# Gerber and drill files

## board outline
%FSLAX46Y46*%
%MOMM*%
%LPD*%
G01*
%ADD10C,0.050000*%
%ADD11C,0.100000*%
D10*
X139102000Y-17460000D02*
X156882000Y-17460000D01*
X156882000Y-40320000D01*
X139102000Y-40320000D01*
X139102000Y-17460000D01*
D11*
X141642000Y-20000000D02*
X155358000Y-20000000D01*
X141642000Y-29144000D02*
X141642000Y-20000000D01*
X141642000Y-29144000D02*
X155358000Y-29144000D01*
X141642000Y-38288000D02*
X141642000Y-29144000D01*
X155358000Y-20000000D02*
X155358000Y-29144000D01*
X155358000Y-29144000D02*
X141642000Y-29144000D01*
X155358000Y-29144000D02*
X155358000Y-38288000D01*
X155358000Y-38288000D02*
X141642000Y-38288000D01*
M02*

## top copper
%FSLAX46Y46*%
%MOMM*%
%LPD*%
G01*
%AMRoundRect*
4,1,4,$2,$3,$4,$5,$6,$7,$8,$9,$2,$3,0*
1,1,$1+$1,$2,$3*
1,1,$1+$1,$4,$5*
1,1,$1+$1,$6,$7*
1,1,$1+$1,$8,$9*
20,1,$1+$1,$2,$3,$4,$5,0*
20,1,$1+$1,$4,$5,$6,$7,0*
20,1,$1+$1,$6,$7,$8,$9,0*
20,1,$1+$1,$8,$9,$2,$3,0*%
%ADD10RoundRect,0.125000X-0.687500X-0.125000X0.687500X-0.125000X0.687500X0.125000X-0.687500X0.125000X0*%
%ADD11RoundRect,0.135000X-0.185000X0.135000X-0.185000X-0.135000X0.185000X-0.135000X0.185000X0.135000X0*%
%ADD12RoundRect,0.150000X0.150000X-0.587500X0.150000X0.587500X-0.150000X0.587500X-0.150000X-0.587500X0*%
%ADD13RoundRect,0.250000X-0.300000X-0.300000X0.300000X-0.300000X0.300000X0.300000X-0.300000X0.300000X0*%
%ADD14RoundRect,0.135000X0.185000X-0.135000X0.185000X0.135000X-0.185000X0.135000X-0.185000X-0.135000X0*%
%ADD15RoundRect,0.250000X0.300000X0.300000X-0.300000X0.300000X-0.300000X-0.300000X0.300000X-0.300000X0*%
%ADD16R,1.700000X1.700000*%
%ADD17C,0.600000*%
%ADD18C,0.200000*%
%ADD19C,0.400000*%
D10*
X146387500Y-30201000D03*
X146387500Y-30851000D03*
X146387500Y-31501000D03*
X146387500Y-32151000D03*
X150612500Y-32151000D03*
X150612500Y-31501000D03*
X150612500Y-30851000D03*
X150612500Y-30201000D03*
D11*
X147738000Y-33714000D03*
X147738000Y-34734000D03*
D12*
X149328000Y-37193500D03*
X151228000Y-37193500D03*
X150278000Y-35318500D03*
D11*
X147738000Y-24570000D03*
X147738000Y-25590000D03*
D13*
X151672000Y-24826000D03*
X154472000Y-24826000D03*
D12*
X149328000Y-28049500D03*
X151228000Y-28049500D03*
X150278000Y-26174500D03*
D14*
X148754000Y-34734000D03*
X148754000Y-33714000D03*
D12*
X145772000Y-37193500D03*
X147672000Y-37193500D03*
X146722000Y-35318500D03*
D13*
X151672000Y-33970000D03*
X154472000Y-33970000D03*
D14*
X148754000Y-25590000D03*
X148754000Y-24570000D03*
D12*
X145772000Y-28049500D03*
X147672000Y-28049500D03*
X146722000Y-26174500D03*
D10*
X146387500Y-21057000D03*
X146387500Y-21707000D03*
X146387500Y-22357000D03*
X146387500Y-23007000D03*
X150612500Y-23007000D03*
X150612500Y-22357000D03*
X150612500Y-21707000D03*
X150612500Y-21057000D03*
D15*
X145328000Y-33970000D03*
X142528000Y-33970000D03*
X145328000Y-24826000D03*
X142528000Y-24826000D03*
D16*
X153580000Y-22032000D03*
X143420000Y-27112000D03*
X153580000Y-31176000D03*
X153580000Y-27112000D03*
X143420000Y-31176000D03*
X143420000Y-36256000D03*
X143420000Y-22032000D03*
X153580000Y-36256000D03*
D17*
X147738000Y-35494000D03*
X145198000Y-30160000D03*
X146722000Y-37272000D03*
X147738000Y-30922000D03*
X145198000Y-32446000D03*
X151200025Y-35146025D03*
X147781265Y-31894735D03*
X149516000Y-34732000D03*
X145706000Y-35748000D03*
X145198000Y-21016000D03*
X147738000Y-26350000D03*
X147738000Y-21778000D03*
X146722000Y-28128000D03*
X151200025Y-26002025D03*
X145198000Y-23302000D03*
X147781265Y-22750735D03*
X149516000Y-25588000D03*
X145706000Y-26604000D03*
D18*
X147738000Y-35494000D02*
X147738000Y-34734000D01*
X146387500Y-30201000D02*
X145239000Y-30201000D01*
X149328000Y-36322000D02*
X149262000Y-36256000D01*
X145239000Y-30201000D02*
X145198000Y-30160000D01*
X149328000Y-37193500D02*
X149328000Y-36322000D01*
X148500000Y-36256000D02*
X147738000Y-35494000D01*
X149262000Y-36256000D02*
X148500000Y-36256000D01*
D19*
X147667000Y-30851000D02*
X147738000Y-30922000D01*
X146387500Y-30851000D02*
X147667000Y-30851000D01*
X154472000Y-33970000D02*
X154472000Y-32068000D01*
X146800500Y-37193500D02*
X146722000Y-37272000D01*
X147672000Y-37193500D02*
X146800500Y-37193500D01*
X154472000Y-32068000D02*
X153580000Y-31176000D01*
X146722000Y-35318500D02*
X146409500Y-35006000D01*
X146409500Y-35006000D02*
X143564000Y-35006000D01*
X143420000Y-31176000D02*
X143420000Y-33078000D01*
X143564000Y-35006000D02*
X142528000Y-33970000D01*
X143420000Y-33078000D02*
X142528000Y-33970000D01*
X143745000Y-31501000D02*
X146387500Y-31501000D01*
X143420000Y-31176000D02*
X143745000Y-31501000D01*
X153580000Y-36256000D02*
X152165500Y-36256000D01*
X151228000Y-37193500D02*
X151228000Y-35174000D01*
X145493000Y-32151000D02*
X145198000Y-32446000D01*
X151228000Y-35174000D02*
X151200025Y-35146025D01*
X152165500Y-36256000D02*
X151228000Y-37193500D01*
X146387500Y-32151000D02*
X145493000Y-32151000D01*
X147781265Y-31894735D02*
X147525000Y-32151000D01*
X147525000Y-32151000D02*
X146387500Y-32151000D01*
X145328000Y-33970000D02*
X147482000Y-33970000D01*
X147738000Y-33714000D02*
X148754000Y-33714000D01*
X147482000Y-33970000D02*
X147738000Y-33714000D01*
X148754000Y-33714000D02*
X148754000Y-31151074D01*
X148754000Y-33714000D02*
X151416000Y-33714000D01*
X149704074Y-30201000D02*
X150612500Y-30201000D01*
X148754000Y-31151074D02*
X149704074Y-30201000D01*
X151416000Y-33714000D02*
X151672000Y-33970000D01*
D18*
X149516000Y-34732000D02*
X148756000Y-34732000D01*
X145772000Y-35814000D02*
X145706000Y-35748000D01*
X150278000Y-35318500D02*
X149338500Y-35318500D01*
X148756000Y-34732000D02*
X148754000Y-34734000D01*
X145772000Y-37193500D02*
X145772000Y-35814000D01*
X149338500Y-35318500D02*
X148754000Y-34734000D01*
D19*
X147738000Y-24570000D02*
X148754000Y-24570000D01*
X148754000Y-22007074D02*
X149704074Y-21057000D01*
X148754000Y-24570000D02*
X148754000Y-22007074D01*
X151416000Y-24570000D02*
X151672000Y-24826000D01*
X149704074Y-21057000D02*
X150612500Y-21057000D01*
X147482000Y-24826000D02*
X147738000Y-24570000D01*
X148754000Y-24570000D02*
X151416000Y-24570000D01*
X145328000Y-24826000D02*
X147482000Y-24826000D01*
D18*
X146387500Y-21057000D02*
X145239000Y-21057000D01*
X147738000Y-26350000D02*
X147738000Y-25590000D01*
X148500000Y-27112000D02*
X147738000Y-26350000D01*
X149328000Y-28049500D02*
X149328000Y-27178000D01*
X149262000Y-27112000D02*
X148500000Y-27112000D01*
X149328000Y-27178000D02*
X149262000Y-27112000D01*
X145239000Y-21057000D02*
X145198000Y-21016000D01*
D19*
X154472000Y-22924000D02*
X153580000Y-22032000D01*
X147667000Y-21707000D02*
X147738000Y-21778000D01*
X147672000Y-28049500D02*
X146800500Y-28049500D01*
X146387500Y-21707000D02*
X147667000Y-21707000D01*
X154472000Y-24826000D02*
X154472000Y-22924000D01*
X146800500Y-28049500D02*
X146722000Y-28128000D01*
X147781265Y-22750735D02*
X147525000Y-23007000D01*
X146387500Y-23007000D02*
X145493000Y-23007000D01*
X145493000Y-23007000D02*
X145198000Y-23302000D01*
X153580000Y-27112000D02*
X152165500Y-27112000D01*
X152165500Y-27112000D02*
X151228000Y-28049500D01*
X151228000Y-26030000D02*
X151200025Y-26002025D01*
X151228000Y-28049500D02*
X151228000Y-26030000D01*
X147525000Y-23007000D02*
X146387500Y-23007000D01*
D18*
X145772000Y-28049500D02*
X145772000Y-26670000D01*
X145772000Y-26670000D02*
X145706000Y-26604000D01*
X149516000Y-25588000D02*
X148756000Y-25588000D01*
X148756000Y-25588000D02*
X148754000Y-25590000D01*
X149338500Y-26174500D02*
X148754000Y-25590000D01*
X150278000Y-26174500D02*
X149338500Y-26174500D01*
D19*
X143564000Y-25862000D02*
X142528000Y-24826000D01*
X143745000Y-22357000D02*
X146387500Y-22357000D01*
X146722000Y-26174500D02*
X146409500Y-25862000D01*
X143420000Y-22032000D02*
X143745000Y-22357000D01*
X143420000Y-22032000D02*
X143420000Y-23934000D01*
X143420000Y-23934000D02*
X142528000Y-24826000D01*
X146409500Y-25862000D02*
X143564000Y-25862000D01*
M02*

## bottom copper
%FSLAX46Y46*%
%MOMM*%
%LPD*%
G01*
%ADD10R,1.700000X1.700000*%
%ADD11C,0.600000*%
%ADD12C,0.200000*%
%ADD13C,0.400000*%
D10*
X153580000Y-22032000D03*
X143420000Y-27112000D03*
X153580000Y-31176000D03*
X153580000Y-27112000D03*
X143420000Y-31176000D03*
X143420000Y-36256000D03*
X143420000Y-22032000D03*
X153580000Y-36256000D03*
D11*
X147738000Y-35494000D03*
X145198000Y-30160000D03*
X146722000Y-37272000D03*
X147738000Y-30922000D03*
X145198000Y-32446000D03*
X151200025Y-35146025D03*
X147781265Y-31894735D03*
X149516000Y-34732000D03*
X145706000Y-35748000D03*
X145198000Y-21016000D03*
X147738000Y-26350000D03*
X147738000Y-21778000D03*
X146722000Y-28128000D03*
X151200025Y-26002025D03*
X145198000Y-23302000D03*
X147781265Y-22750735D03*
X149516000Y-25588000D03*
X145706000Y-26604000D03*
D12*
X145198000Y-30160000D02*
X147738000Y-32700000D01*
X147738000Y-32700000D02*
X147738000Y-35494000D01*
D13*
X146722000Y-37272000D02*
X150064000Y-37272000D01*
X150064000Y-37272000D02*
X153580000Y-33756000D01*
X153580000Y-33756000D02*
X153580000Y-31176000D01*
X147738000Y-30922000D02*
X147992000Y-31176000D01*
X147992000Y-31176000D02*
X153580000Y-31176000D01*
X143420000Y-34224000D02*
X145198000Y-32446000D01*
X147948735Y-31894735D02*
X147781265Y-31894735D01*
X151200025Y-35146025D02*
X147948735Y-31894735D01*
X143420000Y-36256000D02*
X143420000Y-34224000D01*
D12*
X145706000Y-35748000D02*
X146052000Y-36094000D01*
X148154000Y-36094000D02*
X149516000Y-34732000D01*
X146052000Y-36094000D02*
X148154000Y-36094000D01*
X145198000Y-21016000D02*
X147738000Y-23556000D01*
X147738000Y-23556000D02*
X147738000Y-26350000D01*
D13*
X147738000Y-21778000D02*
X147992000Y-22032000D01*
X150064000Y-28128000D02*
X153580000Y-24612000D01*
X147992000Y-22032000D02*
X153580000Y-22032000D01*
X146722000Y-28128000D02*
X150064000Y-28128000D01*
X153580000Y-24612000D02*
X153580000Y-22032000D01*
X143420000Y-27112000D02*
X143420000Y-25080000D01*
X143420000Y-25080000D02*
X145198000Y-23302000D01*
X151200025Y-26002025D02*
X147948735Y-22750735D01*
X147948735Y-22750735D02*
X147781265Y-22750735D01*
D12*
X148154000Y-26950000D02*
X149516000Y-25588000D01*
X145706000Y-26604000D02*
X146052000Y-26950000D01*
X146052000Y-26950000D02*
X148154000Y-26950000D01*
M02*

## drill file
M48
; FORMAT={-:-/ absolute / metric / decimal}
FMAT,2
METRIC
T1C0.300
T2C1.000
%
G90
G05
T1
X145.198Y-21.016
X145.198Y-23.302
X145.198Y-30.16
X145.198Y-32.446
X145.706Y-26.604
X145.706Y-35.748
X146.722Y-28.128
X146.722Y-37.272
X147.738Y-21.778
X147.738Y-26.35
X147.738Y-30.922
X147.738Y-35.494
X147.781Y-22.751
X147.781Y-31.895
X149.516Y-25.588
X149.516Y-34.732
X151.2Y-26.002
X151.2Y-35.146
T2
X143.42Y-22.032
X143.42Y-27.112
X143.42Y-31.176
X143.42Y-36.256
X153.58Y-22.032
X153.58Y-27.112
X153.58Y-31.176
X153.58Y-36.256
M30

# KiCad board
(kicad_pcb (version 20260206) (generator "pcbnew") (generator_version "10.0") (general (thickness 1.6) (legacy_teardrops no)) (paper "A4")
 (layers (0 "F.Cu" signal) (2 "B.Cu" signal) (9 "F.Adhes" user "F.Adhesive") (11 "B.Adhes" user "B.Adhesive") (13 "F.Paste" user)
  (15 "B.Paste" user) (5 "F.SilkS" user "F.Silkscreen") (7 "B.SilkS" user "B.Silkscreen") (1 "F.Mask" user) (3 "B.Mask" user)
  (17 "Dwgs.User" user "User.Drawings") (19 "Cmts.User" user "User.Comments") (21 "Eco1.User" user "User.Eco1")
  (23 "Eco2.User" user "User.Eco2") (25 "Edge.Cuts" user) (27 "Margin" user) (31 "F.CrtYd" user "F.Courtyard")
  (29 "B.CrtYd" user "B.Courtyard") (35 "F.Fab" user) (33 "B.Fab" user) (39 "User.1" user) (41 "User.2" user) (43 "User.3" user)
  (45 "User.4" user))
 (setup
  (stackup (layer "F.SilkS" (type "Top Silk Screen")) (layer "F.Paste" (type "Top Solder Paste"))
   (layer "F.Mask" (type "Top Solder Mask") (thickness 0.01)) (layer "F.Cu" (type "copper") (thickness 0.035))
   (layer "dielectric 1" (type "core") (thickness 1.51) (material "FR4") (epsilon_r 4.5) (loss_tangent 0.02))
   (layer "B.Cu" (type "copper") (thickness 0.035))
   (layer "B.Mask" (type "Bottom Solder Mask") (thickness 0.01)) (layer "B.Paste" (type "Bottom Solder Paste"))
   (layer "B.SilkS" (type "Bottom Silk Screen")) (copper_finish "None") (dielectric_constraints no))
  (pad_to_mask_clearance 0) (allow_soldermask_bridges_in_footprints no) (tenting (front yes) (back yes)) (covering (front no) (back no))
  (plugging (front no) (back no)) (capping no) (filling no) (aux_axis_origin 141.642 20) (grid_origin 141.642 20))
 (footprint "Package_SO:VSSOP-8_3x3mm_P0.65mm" (layer "F.Cu") (at 148.5 31.176)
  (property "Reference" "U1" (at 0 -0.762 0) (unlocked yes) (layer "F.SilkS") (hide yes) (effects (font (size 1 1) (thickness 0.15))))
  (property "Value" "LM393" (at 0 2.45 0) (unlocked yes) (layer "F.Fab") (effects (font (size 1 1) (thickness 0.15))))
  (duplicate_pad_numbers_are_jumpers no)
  (pad "1" smd roundrect (at -2.1125 -0.975) (size 1.625 0.5) (layers "F.Cu" "F.Mask" "F.Paste") (roundrect_rratio 0.25)
   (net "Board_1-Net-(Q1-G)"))
  (pad "2" smd roundrect (at -2.1125 -0.325) (size 1.625 0.5) (layers "F.Cu" "F.Mask" "F.Paste") (roundrect_rratio 0.25) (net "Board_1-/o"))
  (pad "3" smd roundrect (at -2.1125 0.325) (size 1.625 0.5) (layers "F.Cu" "F.Mask" "F.Paste") (roundrect_rratio 0.25) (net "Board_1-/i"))
  (pad "4" smd roundrect (at -2.1125 0.975) (size 1.625 0.5) (layers "F.Cu" "F.Mask" "F.Paste") (roundrect_rratio 0.25) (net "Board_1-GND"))
  (pad "5" smd roundrect (at 2.1125 0.975) (size 1.625 0.5) (layers "F.Cu" "F.Mask" "F.Paste") (roundrect_rratio 0.25)
   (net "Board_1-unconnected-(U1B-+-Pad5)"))
  (pad "6" smd roundrect (at 2.1125 0.325) (size 1.625 0.5) (layers "F.Cu" "F.Mask" "F.Paste") (roundrect_rratio 0.25)
   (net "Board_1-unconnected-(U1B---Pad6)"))
  (pad "7" smd roundrect (at 2.1125 -0.325) (size 1.625 0.5) (layers "F.Cu" "F.Mask" "F.Paste") (roundrect_rratio 0.25)
   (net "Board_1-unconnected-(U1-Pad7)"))
  (pad "8" smd roundrect (at 2.1125 -0.975) (size 1.625 0.5) (layers "F.Cu" "F.Mask" "F.Paste") (roundrect_rratio 0.25) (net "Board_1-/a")))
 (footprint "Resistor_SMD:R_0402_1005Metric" (layer "F.Cu") (at 147.738 34.224 -90)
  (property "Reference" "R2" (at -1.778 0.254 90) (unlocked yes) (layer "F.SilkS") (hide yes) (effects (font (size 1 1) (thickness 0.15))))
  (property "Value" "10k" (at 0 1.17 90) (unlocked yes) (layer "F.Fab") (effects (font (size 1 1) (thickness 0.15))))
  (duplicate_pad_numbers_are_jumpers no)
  (pad "1" smd roundrect (at -0.51 0 270) (size 0.54 0.64) (layers "F.Cu" "F.Mask" "F.Paste") (roundrect_rratio 0.25) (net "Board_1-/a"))
  (pad "2" smd roundrect (at 0.51 0 270) (size 0.54 0.64) (layers "F.Cu" "F.Mask" "F.Paste") (roundrect_rratio 0.25)
   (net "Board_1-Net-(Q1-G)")))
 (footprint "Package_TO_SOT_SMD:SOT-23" (layer "F.Cu") (at 150.278 36.256 90)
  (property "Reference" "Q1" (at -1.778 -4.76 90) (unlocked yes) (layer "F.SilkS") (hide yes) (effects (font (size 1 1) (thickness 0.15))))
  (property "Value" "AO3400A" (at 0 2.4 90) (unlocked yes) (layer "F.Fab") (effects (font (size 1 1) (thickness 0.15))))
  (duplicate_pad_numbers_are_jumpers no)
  (pad "1" smd roundrect (at -0.9375 -0.95 90) (size 1.475 0.6) (layers "F.Cu" "F.Mask" "F.Paste") (roundrect_rratio 0.25)
   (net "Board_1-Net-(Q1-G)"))
  (pad "2" smd roundrect (at -0.9375 0.95 90) (size 1.475 0.6) (layers "F.Cu" "F.Mask" "F.Paste") (roundrect_rratio 0.25)
   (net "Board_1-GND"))
  (pad "3" smd roundrect (at 0.9375 0 90) (size 1.475 0.6) (layers "F.Cu" "F.Mask" "F.Paste") (roundrect_rratio 0.25)
   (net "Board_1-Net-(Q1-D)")))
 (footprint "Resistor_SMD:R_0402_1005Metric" (layer "F.Cu") (at 147.738 25.08 -90)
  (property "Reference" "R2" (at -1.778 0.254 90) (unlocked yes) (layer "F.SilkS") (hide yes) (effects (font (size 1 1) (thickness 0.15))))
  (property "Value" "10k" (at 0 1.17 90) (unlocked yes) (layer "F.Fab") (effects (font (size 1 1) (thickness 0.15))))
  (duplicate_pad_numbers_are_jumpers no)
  (pad "1" smd roundrect (at -0.51 0 270) (size 0.54 0.64) (layers "F.Cu" "F.Mask" "F.Paste") (roundrect_rratio 0.25) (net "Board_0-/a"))
  (pad "2" smd roundrect (at 0.51 0 270) (size 0.54 0.64) (layers "F.Cu" "F.Mask" "F.Paste") (roundrect_rratio 0.25)
   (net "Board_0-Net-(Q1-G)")))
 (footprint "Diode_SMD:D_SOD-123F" (layer "F.Cu") (at 153.072 24.826)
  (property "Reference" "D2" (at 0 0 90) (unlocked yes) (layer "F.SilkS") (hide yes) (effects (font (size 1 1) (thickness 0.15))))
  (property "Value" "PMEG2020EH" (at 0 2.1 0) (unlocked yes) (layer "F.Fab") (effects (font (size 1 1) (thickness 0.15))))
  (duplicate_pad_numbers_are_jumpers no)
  (pad "1" smd roundrect (at -1.4 0) (size 1.1 1.1) (layers "F.Cu" "F.Mask" "F.Paste") (roundrect_rratio 0.2272727273) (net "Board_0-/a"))
  (pad "2" smd roundrect (at 1.4 0) (size 1.1 1.1) (layers "F.Cu" "F.Mask" "F.Paste") (roundrect_rratio 0.2272727273) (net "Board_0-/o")))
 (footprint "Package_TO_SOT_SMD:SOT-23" (layer "F.Cu") (at 150.278 27.112 90)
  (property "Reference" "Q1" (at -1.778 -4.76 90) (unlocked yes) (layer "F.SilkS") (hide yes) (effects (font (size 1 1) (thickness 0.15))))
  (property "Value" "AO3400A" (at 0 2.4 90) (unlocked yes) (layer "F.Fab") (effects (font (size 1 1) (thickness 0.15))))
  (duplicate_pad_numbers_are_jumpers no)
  (pad "1" smd roundrect (at -0.9375 -0.95 90) (size 1.475 0.6) (layers "F.Cu" "F.Mask" "F.Paste") (roundrect_rratio 0.25)
   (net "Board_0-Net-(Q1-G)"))
  (pad "2" smd roundrect (at -0.9375 0.95 90) (size 1.475 0.6) (layers "F.Cu" "F.Mask" "F.Paste") (roundrect_rratio 0.25)
   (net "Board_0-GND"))
  (pad "3" smd roundrect (at 0.9375 0 90) (size 1.475 0.6) (layers "F.Cu" "F.Mask" "F.Paste") (roundrect_rratio 0.25)
   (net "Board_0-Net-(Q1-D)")))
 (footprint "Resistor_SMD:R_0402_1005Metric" (layer "F.Cu") (at 148.754 34.224 90)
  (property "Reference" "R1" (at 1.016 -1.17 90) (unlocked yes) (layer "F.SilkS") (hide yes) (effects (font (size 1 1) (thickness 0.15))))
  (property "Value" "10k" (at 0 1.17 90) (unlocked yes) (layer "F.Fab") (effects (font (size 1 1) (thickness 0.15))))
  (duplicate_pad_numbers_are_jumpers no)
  (pad "1" smd roundrect (at -0.51 0 90) (size 0.54 0.64) (layers "F.Cu" "F.Mask" "F.Paste") (roundrect_rratio 0.25)
   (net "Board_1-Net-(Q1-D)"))
  (pad "2" smd roundrect (at 0.51 0 90) (size 0.54 0.64) (layers "F.Cu" "F.Mask" "F.Paste") (roundrect_rratio 0.25) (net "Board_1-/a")))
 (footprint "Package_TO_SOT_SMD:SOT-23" (layer "F.Cu") (at 146.722 36.256 90)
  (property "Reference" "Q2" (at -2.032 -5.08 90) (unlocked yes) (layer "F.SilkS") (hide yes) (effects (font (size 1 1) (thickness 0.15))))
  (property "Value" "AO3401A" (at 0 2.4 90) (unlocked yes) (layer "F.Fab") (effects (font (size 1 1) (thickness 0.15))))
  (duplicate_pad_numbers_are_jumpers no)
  (pad "1" smd roundrect (at -0.9375 -0.95 90) (size 1.475 0.6) (layers "F.Cu" "F.Mask" "F.Paste") (roundrect_rratio 0.25)
   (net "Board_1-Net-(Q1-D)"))
  (pad "2" smd roundrect (at -0.9375 0.95 90) (size 1.475 0.6) (layers "F.Cu" "F.Mask" "F.Paste") (roundrect_rratio 0.25) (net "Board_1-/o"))
  (pad "3" smd roundrect (at 0.9375 0 90) (size 1.475 0.6) (layers "F.Cu" "F.Mask" "F.Paste") (roundrect_rratio 0.25) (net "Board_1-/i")))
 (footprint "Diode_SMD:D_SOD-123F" (layer "F.Cu") (at 153.072 33.97)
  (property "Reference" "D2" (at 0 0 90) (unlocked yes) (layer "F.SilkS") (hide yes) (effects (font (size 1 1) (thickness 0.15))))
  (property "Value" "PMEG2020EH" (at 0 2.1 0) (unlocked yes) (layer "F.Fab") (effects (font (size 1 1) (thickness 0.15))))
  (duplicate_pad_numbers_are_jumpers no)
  (pad "1" smd roundrect (at -1.4 0) (size 1.1 1.1) (layers "F.Cu" "F.Mask" "F.Paste") (roundrect_rratio 0.2272727273) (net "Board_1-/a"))
  (pad "2" smd roundrect (at 1.4 0) (size 1.1 1.1) (layers "F.Cu" "F.Mask" "F.Paste") (roundrect_rratio 0.2272727273) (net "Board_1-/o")))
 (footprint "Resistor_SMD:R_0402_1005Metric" (layer "F.Cu") (at 148.754 25.08 90)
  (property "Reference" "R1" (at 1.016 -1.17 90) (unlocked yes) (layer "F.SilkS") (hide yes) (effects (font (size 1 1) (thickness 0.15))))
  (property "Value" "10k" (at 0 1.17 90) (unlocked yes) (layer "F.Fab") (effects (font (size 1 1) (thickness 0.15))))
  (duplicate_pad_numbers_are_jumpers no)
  (pad "1" smd roundrect (at -0.51 0 90) (size 0.54 0.64) (layers "F.Cu" "F.Mask" "F.Paste") (roundrect_rratio 0.25)
   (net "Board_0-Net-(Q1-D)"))
  (pad "2" smd roundrect (at 0.51 0 90) (size 0.54 0.64) (layers "F.Cu" "F.Mask" "F.Paste") (roundrect_rratio 0.25) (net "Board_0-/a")))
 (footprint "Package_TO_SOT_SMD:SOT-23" (layer "F.Cu") (at 146.722 27.112 90)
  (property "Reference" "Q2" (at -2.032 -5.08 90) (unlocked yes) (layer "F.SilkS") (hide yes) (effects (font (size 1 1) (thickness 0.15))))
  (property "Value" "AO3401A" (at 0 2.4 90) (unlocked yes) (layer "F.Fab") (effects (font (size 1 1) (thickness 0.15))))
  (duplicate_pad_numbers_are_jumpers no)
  (pad "1" smd roundrect (at -0.9375 -0.95 90) (size 1.475 0.6) (layers "F.Cu" "F.Mask" "F.Paste") (roundrect_rratio 0.25)
   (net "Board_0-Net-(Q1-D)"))
  (pad "2" smd roundrect (at -0.9375 0.95 90) (size 1.475 0.6) (layers "F.Cu" "F.Mask" "F.Paste") (roundrect_rratio 0.25) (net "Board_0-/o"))
  (pad "3" smd roundrect (at 0.9375 0 90) (size 1.475 0.6) (layers "F.Cu" "F.Mask" "F.Paste") (roundrect_rratio 0.25) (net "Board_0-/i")))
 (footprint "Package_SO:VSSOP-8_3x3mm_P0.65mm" (layer "F.Cu") (at 148.5 22.032)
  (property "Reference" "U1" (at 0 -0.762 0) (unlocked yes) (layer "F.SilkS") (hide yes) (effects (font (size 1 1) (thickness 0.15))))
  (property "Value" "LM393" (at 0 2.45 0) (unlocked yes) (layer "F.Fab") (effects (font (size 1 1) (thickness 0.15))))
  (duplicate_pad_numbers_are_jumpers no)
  (pad "1" smd roundrect (at -2.1125 -0.975) (size 1.625 0.5) (layers "F.Cu" "F.Mask" "F.Paste") (roundrect_rratio 0.25)
   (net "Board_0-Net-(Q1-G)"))
  (pad "2" smd roundrect (at -2.1125 -0.325) (size 1.625 0.5) (layers "F.Cu" "F.Mask" "F.Paste") (roundrect_rratio 0.25) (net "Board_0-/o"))
  (pad "3" smd roundrect (at -2.1125 0.325) (size 1.625 0.5) (layers "F.Cu" "F.Mask" "F.Paste") (roundrect_rratio 0.25) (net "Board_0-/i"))
  (pad "4" smd roundrect (at -2.1125 0.975) (size 1.625 0.5) (layers "F.Cu" "F.Mask" "F.Paste") (roundrect_rratio 0.25) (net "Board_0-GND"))
  (pad "5" smd roundrect (at 2.1125 0.975) (size 1.625 0.5) (layers "F.Cu" "F.Mask" "F.Paste") (roundrect_rratio 0.25)
   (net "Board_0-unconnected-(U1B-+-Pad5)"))
  (pad "6" smd roundrect (at 2.1125 0.325) (size 1.625 0.5) (layers "F.Cu" "F.Mask" "F.Paste") (roundrect_rratio 0.25)
   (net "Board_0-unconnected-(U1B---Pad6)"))
  (pad "7" smd roundrect (at 2.1125 -0.325) (size 1.625 0.5) (layers "F.Cu" "F.Mask" "F.Paste") (roundrect_rratio 0.25)
   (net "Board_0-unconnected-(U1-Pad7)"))
  (pad "8" smd roundrect (at 2.1125 -0.975) (size 1.625 0.5) (layers "F.Cu" "F.Mask" "F.Paste") (roundrect_rratio 0.25) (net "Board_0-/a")))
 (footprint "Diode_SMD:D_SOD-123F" (layer "F.Cu") (at 143.928 33.97 180)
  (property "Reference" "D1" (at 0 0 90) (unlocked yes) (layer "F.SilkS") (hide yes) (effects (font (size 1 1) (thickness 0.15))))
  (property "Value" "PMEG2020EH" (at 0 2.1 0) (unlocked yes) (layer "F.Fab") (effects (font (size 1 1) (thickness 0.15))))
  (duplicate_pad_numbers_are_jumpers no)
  (pad "1" smd roundrect (at -1.4 0 180) (size 1.1 1.1) (layers "F.Cu" "F.Mask" "F.Paste") (roundrect_rratio 0.2272727273)
   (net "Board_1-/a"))
  (pad "2" smd roundrect (at 1.4 0 180) (size 1.1 1.1) (layers "F.Cu" "F.Mask" "F.Paste") (roundrect_rratio 0.2272727273) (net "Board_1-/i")))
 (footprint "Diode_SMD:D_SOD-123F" (layer "F.Cu") (at 143.928 24.826 180)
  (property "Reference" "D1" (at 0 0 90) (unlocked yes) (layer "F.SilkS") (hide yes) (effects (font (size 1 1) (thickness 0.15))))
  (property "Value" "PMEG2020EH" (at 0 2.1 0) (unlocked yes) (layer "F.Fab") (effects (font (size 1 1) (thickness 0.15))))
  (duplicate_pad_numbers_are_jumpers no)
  (pad "1" smd roundrect (at -1.4 0 180) (size 1.1 1.1) (layers "F.Cu" "F.Mask" "F.Paste") (roundrect_rratio 0.2272727273)
   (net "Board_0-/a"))
  (pad "2" smd roundrect (at 1.4 0 180) (size 1.1 1.1) (layers "F.Cu" "F.Mask" "F.Paste") (roundrect_rratio 0.2272727273) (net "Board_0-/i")))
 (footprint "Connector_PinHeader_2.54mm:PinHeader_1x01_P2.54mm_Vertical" (layer "B.Cu") (at 153.58 22.032 180)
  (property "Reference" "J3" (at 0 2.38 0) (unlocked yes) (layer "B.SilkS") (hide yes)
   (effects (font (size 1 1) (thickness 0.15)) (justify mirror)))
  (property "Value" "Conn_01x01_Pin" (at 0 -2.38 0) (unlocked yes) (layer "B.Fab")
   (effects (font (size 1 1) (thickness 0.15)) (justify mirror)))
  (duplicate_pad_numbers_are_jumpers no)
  (pad "1" thru_hole rect (at 0 0 180) (size 1.7 1.7) (drill 1) (layers "*.Cu" "*.Mask") (remove_unused_layers no) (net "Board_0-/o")))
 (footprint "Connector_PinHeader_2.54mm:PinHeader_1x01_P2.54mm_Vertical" (layer "B.Cu") (at 143.42 27.112 180)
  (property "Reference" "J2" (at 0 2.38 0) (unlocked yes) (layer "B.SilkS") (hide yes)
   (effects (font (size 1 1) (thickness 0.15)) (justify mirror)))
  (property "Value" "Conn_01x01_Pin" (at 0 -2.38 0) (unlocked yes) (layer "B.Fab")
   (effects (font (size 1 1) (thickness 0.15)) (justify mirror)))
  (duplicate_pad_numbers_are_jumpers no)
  (pad "1" thru_hole rect (at 0 0 180) (size 1.7 1.7) (drill 1) (layers "*.Cu" "*.Mask") (remove_unused_layers no) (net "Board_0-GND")))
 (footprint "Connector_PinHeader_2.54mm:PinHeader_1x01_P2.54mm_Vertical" (layer "B.Cu") (at 153.58 31.176 180)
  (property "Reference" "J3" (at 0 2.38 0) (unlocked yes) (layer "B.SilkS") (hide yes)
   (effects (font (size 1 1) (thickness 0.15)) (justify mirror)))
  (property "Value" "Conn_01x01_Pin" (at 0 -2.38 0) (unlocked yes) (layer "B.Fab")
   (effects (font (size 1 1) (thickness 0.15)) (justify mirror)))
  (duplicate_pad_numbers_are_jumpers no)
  (pad "1" thru_hole rect (at 0 0 180) (size 1.7 1.7) (drill 1) (layers "*.Cu" "*.Mask") (remove_unused_layers no) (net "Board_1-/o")))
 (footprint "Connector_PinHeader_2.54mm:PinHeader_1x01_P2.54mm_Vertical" (layer "B.Cu") (at 153.58 27.112 180)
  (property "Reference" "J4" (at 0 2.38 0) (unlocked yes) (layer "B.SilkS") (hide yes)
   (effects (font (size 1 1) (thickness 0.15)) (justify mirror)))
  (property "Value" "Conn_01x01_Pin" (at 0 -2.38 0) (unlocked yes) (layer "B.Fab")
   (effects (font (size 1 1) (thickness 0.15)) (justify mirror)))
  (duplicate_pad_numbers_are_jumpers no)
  (pad "1" thru_hole rect (at 0 0 180) (size 1.7 1.7) (drill 1) (layers "*.Cu" "*.Mask") (remove_unused_layers no) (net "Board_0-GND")))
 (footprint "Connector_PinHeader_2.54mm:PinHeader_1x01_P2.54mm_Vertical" (layer "B.Cu") (at 143.42 31.176 180)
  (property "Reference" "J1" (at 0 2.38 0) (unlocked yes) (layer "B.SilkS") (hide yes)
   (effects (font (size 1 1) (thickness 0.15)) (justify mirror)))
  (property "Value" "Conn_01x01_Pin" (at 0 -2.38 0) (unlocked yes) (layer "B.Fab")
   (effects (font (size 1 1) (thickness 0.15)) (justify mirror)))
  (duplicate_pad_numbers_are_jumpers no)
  (pad "1" thru_hole rect (at 0 0 180) (size 1.7 1.7) (drill 1) (layers "*.Cu" "*.Mask") (remove_unused_layers no) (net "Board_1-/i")))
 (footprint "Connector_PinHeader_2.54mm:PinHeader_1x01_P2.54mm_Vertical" (layer "B.Cu") (at 143.42 36.256 180)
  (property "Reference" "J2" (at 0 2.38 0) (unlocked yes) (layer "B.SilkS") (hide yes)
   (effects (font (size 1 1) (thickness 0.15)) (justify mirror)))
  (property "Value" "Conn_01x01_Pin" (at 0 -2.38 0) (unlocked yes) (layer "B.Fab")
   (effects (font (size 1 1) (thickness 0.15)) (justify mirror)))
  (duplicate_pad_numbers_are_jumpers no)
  (pad "1" thru_hole rect (at 0 0 180) (size 1.7 1.7) (drill 1) (layers "*.Cu" "*.Mask") (remove_unused_layers no) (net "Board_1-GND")))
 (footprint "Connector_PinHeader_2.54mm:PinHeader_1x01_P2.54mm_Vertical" (layer "B.Cu") (at 143.42 22.032 180)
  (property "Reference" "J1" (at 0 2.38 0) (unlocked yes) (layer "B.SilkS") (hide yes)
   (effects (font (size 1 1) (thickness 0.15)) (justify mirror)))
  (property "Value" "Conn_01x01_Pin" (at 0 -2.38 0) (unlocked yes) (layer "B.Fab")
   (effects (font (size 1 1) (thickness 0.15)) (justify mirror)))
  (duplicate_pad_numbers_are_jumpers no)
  (pad "1" thru_hole rect (at 0 0 180) (size 1.7 1.7) (drill 1) (layers "*.Cu" "*.Mask") (remove_unused_layers no) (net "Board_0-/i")))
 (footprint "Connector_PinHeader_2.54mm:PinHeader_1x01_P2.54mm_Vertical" (layer "B.Cu") (at 153.58 36.256 180)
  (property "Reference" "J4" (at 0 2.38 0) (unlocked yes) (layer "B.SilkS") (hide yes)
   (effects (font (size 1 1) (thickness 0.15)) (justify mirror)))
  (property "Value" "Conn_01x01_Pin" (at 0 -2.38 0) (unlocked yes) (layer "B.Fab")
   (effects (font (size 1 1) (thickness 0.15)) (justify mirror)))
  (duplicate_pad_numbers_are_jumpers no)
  (pad "1" thru_hole rect (at 0 0 180) (size 1.7 1.7) (drill 1) (layers "*.Cu" "*.Mask") (remove_unused_layers no) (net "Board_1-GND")))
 (gr_rect (start 139.102 17.46) (end 156.882 40.32) (stroke (width 0.05) (type default)) (fill no) (layer "Edge.Cuts"))
 (gr_line (start 141.642 20) (end 155.358 20) (stroke (width 0.1) (type default)) (layer "Edge.Cuts"))
 (gr_line (start 141.642 29.144) (end 141.642 20) (stroke (width 0.1) (type default)) (layer "Edge.Cuts"))
 (gr_line (start 141.642 29.144) (end 155.358 29.144) (stroke (width 0.1) (type default)) (layer "Edge.Cuts"))
 (gr_line (start 141.642 38.288) (end 141.642 29.144) (stroke (width 0.1) (type default)) (layer "Edge.Cuts"))
 (gr_line (start 155.358 20) (end 155.358 29.144) (stroke (width 0.1) (type default)) (layer "Edge.Cuts"))
 (gr_line (start 155.358 29.144) (end 141.642 29.144) (stroke (width 0.1) (type default)) (layer "Edge.Cuts"))
 (gr_line (start 155.358 29.144) (end 155.358 38.288) (stroke (width 0.1) (type default)) (layer "Edge.Cuts"))
 (gr_line (start 155.358 38.288) (end 141.642 38.288) (stroke (width 0.1) (type default)) (layer "Edge.Cuts"))
 (segment (start 147.738 35.494) (end 147.738 34.734) (width 0.2) (layer "F.Cu") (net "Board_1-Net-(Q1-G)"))
 (segment (start 146.3875 30.201) (end 145.239 30.201) (width 0.2) (layer "F.Cu") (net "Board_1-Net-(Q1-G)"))
 (segment (start 149.328 36.322) (end 149.262 36.256) (width 0.2) (layer "F.Cu") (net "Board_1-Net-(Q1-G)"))
 (segment (start 145.239 30.201) (end 145.198 30.16) (width 0.2) (layer "F.Cu") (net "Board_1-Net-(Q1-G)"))
 (segment (start 149.328 37.1935) (end 149.328 36.322) (width 0.2) (layer "F.Cu") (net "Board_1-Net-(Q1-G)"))
 (segment (start 148.5 36.256) (end 147.738 35.494) (width 0.2) (layer "F.Cu") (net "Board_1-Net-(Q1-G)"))
 (segment (start 149.262 36.256) (end 148.5 36.256) (width 0.2) (layer "F.Cu") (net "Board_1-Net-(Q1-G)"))
 (via (at 147.738 35.494) (size 0.6) (drill 0.3) (layers "F.Cu" "B.Cu") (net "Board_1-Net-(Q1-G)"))
 (via (at 145.198 30.16) (size 0.6) (drill 0.3) (layers "F.Cu" "B.Cu") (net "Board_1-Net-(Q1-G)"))
 (segment (start 145.198 30.16) (end 147.738 32.7) (width 0.2) (layer "B.Cu") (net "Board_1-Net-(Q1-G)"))
 (segment (start 147.738 32.7) (end 147.738 35.494) (width 0.2) (layer "B.Cu") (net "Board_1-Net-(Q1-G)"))
 (segment (start 147.667 30.851) (end 147.738 30.922) (width 0.4) (layer "F.Cu") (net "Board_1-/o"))
 (segment (start 146.3875 30.851) (end 147.667 30.851) (width 0.4) (layer "F.Cu") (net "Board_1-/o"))
 (segment (start 154.472 33.97) (end 154.472 32.068) (width 0.4) (layer "F.Cu") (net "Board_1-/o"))
 (segment (start 146.8005 37.1935) (end 146.722 37.272) (width 0.4) (layer "F.Cu") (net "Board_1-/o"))
 (segment (start 147.672 37.1935) (end 146.8005 37.1935) (width 0.4) (layer "F.Cu") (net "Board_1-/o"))
 (segment (start 154.472 32.068) (end 153.58 31.176) (width 0.4) (layer "F.Cu") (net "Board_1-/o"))
 (via (at 146.722 37.272) (size 0.6) (drill 0.3) (layers "F.Cu" "B.Cu") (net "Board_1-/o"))
 (via (at 147.738 30.922) (size 0.6) (drill 0.3) (layers "F.Cu" "B.Cu") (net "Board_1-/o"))
 (segment (start 146.722 37.272) (end 150.064 37.272) (width 0.4) (layer "B.Cu") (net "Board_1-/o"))
 (segment (start 150.064 37.272) (end 153.58 33.756) (width 0.4) (layer "B.Cu") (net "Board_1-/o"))
 (segment (start 153.58 33.756) (end 153.58 31.176) (width 0.4) (layer "B.Cu") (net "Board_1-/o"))
 (segment (start 147.738 30.922) (end 147.992 31.176) (width 0.4) (layer "B.Cu") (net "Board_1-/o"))
 (segment (start 147.992 31.176) (end 153.58 31.176) (width 0.4) (layer "B.Cu") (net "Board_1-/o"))
 (segment (start 146.722 35.3185) (end 146.4095 35.006) (width 0.4) (layer "F.Cu") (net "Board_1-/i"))
 (segment (start 146.4095 35.006) (end 143.564 35.006) (width 0.4) (layer "F.Cu") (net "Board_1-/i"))
 (segment (start 143.42 31.176) (end 143.42 33.078) (width 0.4) (layer "F.Cu") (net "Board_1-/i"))
 (segment (start 143.564 35.006) (end 142.528 33.97) (width 0.4) (layer "F.Cu") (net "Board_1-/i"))
 (segment (start 143.42 33.078) (end 142.528 33.97) (width 0.4) (layer "F.Cu") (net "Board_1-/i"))
 (segment (start 143.745 31.501) (end 146.3875 31.501) (width 0.4) (layer "F.Cu") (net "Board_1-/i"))
 (segment (start 143.42 31.176) (end 143.745 31.501) (width 0.4) (layer "F.Cu") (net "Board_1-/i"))
 (segment (start 153.58 36.256) (end 152.1655 36.256) (width 0.4) (layer "F.Cu") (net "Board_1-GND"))
 (segment (start 151.228 37.1935) (end 151.228 35.174) (width 0.4) (layer "F.Cu") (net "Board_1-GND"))
 (segment (start 145.493 32.151) (end 145.198 32.446) (width 0.4) (layer "F.Cu") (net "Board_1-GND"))
 (segment (start 151.228 35.174) (end 151.200025 35.146025) (width 0.4) (layer "F.Cu") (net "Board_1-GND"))
 (segment (start 152.1655 36.256) (end 151.228 37.1935) (width 0.4) (layer "F.Cu") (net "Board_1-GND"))
 (segment (start 146.3875 32.151) (end 145.493 32.151) (width 0.4) (layer "F.Cu") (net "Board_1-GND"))
 (segment (start 147.781265 31.894735) (end 147.525 32.151) (width 0.4) (layer "F.Cu") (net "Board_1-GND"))
 (segment (start 147.525 32.151) (end 146.3875 32.151) (width 0.4) (layer "F.Cu") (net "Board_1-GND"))
 (via blind (at 145.198 32.446) (size 0.6) (drill 0.3) (layers "F.Cu" "B.Cu") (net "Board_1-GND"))
 (via (at 151.200025 35.146025) (size 0.6) (drill 0.3) (layers "F.Cu" "B.Cu") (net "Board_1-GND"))
 (via (at 147.781265 31.894735) (size 0.6) (drill 0.3) (layers "F.Cu" "B.Cu") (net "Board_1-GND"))
 (segment (start 143.42 34.224) (end 145.198 32.446) (width 0.4) (layer "B.Cu") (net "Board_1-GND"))
 (segment (start 147.948735 31.894735) (end 147.781265 31.894735) (width 0.4) (layer "B.Cu") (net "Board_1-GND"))
 (segment (start 151.200025 35.146025) (end 147.948735 31.894735) (width 0.4) (layer "B.Cu") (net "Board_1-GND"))
 (segment (start 143.42 36.256) (end 143.42 34.224) (width 0.4) (layer "B.Cu") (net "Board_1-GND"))
 (segment (start 145.328 33.97) (end 147.482 33.97) (width 0.4) (layer "F.Cu") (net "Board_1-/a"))
 (segment (start 147.738 33.714) (end 148.754 33.714) (width 0.4) (layer "F.Cu") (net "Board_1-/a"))
 (segment (start 147.482 33.97) (end 147.738 33.714) (width 0.4) (layer "F.Cu") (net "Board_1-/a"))
 (segment (start 148.754 33.714) (end 148.754 31.151074) (width 0.4) (layer "F.Cu") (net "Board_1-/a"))
 (segment (start 148.754 33.714) (end 151.416 33.714) (width 0.4) (layer "F.Cu") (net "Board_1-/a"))
 (segment (start 149.704074 30.201) (end 150.6125 30.201) (width 0.4) (layer "F.Cu") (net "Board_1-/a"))
 (segment (start 148.754 31.151074) (end 149.704074 30.201) (width 0.4) (layer "F.Cu") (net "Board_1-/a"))
 (segment (start 151.416 33.714) (end 151.672 33.97) (width 0.4) (layer "F.Cu") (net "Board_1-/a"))
 (segment (start 149.516 34.732) (end 148.756 34.732) (width 0.2) (layer "F.Cu") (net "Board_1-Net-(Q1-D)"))
 (segment (start 145.772 35.814) (end 145.706 35.748) (width 0.2) (layer "F.Cu") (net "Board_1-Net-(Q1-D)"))
 (segment (start 150.278 35.3185) (end 149.3385 35.3185) (width 0.2) (layer "F.Cu") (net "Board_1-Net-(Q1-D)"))
 (segment (start 148.756 34.732) (end 148.754 34.734) (width 0.2) (layer "F.Cu") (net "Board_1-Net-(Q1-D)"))
 (segment (start 145.772 37.1935) (end 145.772 35.814) (width 0.2) (layer "F.Cu") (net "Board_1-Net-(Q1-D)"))
 (segment (start 149.3385 35.3185) (end 148.754 34.734) (width 0.2) (layer "F.Cu") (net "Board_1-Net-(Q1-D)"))
 (via (at 149.516 34.732) (size 0.6) (drill 0.3) (layers "F.Cu" "B.Cu") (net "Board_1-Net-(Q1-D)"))
 (via (at 145.706 35.748) (size 0.6) (drill 0.3) (layers "F.Cu" "B.Cu") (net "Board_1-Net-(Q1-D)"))
 (segment (start 145.706 35.748) (end 146.052 36.094) (width 0.2) (layer "B.Cu") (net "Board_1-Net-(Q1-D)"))
 (segment (start 148.154 36.094) (end 149.516 34.732) (width 0.2) (layer "B.Cu") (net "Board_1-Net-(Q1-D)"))
 (segment (start 146.052 36.094) (end 148.154 36.094) (width 0.2) (layer "B.Cu") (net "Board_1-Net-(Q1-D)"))
 (segment (start 147.738 24.57) (end 148.754 24.57) (width 0.4) (layer "F.Cu") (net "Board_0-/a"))
 (segment (start 148.754 22.007074) (end 149.704074 21.057) (width 0.4) (layer "F.Cu") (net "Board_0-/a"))
 (segment (start 148.754 24.57) (end 148.754 22.007074) (width 0.4) (layer "F.Cu") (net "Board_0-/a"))
 (segment (start 151.416 24.57) (end 151.672 24.826) (width 0.4) (layer "F.Cu") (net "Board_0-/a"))
 (segment (start 149.704074 21.057) (end 150.6125 21.057) (width 0.4) (layer "F.Cu") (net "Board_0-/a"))
 (segment (start 147.482 24.826) (end 147.738 24.57) (width 0.4) (layer "F.Cu") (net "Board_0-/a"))
 (segment (start 148.754 24.57) (end 151.416 24.57) (width 0.4) (layer "F.Cu") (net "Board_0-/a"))
 (segment (start 145.328 24.826) (end 147.482 24.826) (width 0.4) (layer "F.Cu") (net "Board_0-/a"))
 (segment (start 146.3875 21.057) (end 145.239 21.057) (width 0.2) (layer "F.Cu") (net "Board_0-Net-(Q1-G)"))
 (segment (start 147.738 26.35) (end 147.738 25.59) (width 0.2) (layer "F.Cu") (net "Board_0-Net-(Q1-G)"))
 (segment (start 148.5 27.112) (end 147.738 26.35) (width 0.2) (layer "F.Cu") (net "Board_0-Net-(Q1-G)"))
 (segment (start 149.328 28.0495) (end 149.328 27.178) (width 0.2) (layer "F.Cu") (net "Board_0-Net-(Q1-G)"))
 (segment (start 149.262 27.112) (end 148.5 27.112) (width 0.2) (layer "F.Cu") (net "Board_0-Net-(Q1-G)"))
 (segment (start 149.328 27.178) (end 149.262 27.112) (width 0.2) (layer "F.Cu") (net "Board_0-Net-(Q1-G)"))
 (segment (start 145.239 21.057) (end 145.198 21.016) (width 0.2) (layer "F.Cu") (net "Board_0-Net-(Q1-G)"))
 (via (at 145.198 21.016) (size 0.6) (drill 0.3) (layers "F.Cu" "B.Cu") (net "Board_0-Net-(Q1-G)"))
 (via (at 147.738 26.35) (size 0.6) (drill 0.3) (layers "F.Cu" "B.Cu") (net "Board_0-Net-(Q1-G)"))
 (segment (start 145.198 21.016) (end 147.738 23.556) (width 0.2) (layer "B.Cu") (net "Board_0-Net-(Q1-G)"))
 (segment (start 147.738 23.556) (end 147.738 26.35) (width 0.2) (layer "B.Cu") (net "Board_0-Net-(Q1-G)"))
 (segment (start 154.472 22.924) (end 153.58 22.032) (width 0.4) (layer "F.Cu") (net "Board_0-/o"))
 (segment (start 147.667 21.707) (end 147.738 21.778) (width 0.4) (layer "F.Cu") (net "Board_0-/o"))
 (segment (start 147.672 28.0495) (end 146.8005 28.0495) (width 0.4) (layer "F.Cu") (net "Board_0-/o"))
 (segment (start 146.3875 21.707) (end 147.667 21.707) (width 0.4) (layer "F.Cu") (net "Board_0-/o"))
 (segment (start 154.472 24.826) (end 154.472 22.924) (width 0.4) (layer "F.Cu") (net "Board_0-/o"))
 (segment (start 146.8005 28.0495) (end 146.722 28.128) (width 0.4) (layer "F.Cu") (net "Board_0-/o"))
 (via (at 147.738 21.778) (size 0.6) (drill 0.3) (layers "F.Cu" "B.Cu") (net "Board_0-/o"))
 (via (at 146.722 28.128) (size 0.6) (drill 0.3) (layers "F.Cu" "B.Cu") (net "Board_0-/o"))
 (segment (start 147.738 21.778) (end 147.992 22.032) (width 0.4) (layer "B.Cu") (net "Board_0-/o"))
 (segment (start 150.064 28.128) (end 153.58 24.612) (width 0.4) (layer "B.Cu") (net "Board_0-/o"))
 (segment (start 147.992 22.032) (end 153.58 22.032) (width 0.4) (layer "B.Cu") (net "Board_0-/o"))
 (segment (start 146.722 28.128) (end 150.064 28.128) (width 0.4) (layer "B.Cu") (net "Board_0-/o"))
 (segment (start 153.58 24.612) (end 153.58 22.032) (width 0.4) (layer "B.Cu") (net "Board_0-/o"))
 (segment (start 147.781265 22.750735) (end 147.525 23.007) (width 0.4) (layer "F.Cu") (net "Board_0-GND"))
 (segment (start 146.3875 23.007) (end 145.493 23.007) (width 0.4) (layer "F.Cu") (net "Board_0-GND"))
 (segment (start 145.493 23.007) (end 145.198 23.302) (width 0.4) (layer "F.Cu") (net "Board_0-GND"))
 (segment (start 153.58 27.112) (end 152.1655 27.112) (width 0.4) (layer "F.Cu") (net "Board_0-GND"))
 (segment (start 152.1655 27.112) (end 151.228 28.0495) (width 0.4) (layer "F.Cu") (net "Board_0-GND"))
 (segment (start 151.228 26.03) (end 151.200025 26.002025) (width 0.4) (layer "F.Cu") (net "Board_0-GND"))
 (segment (start 151.228 28.0495) (end 151.228 26.03) (width 0.4) (layer "F.Cu") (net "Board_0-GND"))
 (segment (start 147.525 23.007) (end 146.3875 23.007) (width 0.4) (layer "F.Cu") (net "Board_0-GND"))
 (via (at 151.200025 26.002025) (size 0.6) (drill 0.3) (layers "F.Cu" "B.Cu") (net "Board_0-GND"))
 (via blind (at 145.198 23.302) (size 0.6) (drill 0.3) (layers "F.Cu" "B.Cu") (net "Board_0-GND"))
 (via (at 147.781265 22.750735) (size 0.6) (drill 0.3) (layers "F.Cu" "B.Cu") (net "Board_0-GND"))
 (segment (start 143.42 27.112) (end 143.42 25.08) (width 0.4) (layer "B.Cu") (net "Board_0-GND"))
 (segment (start 143.42 25.08) (end 145.198 23.302) (width 0.4) (layer "B.Cu") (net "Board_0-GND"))
 (segment (start 151.200025 26.002025) (end 147.948735 22.750735) (width 0.4) (layer "B.Cu") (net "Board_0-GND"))
 (segment (start 147.948735 22.750735) (end 147.781265 22.750735) (width 0.4) (layer "B.Cu") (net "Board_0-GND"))
 (segment (start 145.772 28.0495) (end 145.772 26.67) (width 0.2) (layer "F.Cu") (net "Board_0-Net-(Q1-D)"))
 (segment (start 145.772 26.67) (end 145.706 26.604) (width 0.2) (layer "F.Cu") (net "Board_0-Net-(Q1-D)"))
 (segment (start 149.516 25.588) (end 148.756 25.588) (width 0.2) (layer "F.Cu") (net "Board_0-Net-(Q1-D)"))
 (segment (start 148.756 25.588) (end 148.754 25.59) (width 0.2) (layer "F.Cu") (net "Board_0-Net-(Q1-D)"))
 (segment (start 149.3385 26.1745) (end 148.754 25.59) (width 0.2) (layer "F.Cu") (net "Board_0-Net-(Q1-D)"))
 (segment (start 150.278 26.1745) (end 149.3385 26.1745) (width 0.2) (layer "F.Cu") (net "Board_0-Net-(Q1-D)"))
 (via (at 149.516 25.588) (size 0.6) (drill 0.3) (layers "F.Cu" "B.Cu") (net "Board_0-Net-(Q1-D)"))
 (via (at 145.706 26.604) (size 0.6) (drill 0.3) (layers "F.Cu" "B.Cu") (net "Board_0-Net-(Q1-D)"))
 (segment (start 148.154 26.95) (end 149.516 25.588) (width 0.2) (layer "B.Cu") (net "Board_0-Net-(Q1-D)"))
 (segment (start 145.706 26.604) (end 146.052 26.95) (width 0.2) (layer "B.Cu") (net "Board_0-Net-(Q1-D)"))
 (segment (start 146.052 26.95) (end 148.154 26.95) (width 0.2) (layer "B.Cu") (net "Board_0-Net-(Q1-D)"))
 (segment (start 143.564 25.862) (end 142.528 24.826) (width 0.4) (layer "F.Cu") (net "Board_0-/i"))
 (segment (start 143.745 22.357) (end 146.3875 22.357) (width 0.4) (layer "F.Cu") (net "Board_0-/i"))
 (segment (start 146.722 26.1745) (end 146.4095 25.862) (width 0.4) (layer "F.Cu") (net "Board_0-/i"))
 (segment (start 143.42 22.032) (end 143.745 22.357) (width 0.4) (layer "F.Cu") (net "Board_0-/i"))
 (segment (start 143.42 22.032) (end 143.42 23.934) (width 0.4) (layer "F.Cu") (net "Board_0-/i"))
 (segment (start 143.42 23.934) (end 142.528 24.826) (width 0.4) (layer "F.Cu") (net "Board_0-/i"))
 (segment (start 146.4095 25.862) (end 143.564 25.862) (width 0.4) (layer "F.Cu") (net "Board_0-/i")))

